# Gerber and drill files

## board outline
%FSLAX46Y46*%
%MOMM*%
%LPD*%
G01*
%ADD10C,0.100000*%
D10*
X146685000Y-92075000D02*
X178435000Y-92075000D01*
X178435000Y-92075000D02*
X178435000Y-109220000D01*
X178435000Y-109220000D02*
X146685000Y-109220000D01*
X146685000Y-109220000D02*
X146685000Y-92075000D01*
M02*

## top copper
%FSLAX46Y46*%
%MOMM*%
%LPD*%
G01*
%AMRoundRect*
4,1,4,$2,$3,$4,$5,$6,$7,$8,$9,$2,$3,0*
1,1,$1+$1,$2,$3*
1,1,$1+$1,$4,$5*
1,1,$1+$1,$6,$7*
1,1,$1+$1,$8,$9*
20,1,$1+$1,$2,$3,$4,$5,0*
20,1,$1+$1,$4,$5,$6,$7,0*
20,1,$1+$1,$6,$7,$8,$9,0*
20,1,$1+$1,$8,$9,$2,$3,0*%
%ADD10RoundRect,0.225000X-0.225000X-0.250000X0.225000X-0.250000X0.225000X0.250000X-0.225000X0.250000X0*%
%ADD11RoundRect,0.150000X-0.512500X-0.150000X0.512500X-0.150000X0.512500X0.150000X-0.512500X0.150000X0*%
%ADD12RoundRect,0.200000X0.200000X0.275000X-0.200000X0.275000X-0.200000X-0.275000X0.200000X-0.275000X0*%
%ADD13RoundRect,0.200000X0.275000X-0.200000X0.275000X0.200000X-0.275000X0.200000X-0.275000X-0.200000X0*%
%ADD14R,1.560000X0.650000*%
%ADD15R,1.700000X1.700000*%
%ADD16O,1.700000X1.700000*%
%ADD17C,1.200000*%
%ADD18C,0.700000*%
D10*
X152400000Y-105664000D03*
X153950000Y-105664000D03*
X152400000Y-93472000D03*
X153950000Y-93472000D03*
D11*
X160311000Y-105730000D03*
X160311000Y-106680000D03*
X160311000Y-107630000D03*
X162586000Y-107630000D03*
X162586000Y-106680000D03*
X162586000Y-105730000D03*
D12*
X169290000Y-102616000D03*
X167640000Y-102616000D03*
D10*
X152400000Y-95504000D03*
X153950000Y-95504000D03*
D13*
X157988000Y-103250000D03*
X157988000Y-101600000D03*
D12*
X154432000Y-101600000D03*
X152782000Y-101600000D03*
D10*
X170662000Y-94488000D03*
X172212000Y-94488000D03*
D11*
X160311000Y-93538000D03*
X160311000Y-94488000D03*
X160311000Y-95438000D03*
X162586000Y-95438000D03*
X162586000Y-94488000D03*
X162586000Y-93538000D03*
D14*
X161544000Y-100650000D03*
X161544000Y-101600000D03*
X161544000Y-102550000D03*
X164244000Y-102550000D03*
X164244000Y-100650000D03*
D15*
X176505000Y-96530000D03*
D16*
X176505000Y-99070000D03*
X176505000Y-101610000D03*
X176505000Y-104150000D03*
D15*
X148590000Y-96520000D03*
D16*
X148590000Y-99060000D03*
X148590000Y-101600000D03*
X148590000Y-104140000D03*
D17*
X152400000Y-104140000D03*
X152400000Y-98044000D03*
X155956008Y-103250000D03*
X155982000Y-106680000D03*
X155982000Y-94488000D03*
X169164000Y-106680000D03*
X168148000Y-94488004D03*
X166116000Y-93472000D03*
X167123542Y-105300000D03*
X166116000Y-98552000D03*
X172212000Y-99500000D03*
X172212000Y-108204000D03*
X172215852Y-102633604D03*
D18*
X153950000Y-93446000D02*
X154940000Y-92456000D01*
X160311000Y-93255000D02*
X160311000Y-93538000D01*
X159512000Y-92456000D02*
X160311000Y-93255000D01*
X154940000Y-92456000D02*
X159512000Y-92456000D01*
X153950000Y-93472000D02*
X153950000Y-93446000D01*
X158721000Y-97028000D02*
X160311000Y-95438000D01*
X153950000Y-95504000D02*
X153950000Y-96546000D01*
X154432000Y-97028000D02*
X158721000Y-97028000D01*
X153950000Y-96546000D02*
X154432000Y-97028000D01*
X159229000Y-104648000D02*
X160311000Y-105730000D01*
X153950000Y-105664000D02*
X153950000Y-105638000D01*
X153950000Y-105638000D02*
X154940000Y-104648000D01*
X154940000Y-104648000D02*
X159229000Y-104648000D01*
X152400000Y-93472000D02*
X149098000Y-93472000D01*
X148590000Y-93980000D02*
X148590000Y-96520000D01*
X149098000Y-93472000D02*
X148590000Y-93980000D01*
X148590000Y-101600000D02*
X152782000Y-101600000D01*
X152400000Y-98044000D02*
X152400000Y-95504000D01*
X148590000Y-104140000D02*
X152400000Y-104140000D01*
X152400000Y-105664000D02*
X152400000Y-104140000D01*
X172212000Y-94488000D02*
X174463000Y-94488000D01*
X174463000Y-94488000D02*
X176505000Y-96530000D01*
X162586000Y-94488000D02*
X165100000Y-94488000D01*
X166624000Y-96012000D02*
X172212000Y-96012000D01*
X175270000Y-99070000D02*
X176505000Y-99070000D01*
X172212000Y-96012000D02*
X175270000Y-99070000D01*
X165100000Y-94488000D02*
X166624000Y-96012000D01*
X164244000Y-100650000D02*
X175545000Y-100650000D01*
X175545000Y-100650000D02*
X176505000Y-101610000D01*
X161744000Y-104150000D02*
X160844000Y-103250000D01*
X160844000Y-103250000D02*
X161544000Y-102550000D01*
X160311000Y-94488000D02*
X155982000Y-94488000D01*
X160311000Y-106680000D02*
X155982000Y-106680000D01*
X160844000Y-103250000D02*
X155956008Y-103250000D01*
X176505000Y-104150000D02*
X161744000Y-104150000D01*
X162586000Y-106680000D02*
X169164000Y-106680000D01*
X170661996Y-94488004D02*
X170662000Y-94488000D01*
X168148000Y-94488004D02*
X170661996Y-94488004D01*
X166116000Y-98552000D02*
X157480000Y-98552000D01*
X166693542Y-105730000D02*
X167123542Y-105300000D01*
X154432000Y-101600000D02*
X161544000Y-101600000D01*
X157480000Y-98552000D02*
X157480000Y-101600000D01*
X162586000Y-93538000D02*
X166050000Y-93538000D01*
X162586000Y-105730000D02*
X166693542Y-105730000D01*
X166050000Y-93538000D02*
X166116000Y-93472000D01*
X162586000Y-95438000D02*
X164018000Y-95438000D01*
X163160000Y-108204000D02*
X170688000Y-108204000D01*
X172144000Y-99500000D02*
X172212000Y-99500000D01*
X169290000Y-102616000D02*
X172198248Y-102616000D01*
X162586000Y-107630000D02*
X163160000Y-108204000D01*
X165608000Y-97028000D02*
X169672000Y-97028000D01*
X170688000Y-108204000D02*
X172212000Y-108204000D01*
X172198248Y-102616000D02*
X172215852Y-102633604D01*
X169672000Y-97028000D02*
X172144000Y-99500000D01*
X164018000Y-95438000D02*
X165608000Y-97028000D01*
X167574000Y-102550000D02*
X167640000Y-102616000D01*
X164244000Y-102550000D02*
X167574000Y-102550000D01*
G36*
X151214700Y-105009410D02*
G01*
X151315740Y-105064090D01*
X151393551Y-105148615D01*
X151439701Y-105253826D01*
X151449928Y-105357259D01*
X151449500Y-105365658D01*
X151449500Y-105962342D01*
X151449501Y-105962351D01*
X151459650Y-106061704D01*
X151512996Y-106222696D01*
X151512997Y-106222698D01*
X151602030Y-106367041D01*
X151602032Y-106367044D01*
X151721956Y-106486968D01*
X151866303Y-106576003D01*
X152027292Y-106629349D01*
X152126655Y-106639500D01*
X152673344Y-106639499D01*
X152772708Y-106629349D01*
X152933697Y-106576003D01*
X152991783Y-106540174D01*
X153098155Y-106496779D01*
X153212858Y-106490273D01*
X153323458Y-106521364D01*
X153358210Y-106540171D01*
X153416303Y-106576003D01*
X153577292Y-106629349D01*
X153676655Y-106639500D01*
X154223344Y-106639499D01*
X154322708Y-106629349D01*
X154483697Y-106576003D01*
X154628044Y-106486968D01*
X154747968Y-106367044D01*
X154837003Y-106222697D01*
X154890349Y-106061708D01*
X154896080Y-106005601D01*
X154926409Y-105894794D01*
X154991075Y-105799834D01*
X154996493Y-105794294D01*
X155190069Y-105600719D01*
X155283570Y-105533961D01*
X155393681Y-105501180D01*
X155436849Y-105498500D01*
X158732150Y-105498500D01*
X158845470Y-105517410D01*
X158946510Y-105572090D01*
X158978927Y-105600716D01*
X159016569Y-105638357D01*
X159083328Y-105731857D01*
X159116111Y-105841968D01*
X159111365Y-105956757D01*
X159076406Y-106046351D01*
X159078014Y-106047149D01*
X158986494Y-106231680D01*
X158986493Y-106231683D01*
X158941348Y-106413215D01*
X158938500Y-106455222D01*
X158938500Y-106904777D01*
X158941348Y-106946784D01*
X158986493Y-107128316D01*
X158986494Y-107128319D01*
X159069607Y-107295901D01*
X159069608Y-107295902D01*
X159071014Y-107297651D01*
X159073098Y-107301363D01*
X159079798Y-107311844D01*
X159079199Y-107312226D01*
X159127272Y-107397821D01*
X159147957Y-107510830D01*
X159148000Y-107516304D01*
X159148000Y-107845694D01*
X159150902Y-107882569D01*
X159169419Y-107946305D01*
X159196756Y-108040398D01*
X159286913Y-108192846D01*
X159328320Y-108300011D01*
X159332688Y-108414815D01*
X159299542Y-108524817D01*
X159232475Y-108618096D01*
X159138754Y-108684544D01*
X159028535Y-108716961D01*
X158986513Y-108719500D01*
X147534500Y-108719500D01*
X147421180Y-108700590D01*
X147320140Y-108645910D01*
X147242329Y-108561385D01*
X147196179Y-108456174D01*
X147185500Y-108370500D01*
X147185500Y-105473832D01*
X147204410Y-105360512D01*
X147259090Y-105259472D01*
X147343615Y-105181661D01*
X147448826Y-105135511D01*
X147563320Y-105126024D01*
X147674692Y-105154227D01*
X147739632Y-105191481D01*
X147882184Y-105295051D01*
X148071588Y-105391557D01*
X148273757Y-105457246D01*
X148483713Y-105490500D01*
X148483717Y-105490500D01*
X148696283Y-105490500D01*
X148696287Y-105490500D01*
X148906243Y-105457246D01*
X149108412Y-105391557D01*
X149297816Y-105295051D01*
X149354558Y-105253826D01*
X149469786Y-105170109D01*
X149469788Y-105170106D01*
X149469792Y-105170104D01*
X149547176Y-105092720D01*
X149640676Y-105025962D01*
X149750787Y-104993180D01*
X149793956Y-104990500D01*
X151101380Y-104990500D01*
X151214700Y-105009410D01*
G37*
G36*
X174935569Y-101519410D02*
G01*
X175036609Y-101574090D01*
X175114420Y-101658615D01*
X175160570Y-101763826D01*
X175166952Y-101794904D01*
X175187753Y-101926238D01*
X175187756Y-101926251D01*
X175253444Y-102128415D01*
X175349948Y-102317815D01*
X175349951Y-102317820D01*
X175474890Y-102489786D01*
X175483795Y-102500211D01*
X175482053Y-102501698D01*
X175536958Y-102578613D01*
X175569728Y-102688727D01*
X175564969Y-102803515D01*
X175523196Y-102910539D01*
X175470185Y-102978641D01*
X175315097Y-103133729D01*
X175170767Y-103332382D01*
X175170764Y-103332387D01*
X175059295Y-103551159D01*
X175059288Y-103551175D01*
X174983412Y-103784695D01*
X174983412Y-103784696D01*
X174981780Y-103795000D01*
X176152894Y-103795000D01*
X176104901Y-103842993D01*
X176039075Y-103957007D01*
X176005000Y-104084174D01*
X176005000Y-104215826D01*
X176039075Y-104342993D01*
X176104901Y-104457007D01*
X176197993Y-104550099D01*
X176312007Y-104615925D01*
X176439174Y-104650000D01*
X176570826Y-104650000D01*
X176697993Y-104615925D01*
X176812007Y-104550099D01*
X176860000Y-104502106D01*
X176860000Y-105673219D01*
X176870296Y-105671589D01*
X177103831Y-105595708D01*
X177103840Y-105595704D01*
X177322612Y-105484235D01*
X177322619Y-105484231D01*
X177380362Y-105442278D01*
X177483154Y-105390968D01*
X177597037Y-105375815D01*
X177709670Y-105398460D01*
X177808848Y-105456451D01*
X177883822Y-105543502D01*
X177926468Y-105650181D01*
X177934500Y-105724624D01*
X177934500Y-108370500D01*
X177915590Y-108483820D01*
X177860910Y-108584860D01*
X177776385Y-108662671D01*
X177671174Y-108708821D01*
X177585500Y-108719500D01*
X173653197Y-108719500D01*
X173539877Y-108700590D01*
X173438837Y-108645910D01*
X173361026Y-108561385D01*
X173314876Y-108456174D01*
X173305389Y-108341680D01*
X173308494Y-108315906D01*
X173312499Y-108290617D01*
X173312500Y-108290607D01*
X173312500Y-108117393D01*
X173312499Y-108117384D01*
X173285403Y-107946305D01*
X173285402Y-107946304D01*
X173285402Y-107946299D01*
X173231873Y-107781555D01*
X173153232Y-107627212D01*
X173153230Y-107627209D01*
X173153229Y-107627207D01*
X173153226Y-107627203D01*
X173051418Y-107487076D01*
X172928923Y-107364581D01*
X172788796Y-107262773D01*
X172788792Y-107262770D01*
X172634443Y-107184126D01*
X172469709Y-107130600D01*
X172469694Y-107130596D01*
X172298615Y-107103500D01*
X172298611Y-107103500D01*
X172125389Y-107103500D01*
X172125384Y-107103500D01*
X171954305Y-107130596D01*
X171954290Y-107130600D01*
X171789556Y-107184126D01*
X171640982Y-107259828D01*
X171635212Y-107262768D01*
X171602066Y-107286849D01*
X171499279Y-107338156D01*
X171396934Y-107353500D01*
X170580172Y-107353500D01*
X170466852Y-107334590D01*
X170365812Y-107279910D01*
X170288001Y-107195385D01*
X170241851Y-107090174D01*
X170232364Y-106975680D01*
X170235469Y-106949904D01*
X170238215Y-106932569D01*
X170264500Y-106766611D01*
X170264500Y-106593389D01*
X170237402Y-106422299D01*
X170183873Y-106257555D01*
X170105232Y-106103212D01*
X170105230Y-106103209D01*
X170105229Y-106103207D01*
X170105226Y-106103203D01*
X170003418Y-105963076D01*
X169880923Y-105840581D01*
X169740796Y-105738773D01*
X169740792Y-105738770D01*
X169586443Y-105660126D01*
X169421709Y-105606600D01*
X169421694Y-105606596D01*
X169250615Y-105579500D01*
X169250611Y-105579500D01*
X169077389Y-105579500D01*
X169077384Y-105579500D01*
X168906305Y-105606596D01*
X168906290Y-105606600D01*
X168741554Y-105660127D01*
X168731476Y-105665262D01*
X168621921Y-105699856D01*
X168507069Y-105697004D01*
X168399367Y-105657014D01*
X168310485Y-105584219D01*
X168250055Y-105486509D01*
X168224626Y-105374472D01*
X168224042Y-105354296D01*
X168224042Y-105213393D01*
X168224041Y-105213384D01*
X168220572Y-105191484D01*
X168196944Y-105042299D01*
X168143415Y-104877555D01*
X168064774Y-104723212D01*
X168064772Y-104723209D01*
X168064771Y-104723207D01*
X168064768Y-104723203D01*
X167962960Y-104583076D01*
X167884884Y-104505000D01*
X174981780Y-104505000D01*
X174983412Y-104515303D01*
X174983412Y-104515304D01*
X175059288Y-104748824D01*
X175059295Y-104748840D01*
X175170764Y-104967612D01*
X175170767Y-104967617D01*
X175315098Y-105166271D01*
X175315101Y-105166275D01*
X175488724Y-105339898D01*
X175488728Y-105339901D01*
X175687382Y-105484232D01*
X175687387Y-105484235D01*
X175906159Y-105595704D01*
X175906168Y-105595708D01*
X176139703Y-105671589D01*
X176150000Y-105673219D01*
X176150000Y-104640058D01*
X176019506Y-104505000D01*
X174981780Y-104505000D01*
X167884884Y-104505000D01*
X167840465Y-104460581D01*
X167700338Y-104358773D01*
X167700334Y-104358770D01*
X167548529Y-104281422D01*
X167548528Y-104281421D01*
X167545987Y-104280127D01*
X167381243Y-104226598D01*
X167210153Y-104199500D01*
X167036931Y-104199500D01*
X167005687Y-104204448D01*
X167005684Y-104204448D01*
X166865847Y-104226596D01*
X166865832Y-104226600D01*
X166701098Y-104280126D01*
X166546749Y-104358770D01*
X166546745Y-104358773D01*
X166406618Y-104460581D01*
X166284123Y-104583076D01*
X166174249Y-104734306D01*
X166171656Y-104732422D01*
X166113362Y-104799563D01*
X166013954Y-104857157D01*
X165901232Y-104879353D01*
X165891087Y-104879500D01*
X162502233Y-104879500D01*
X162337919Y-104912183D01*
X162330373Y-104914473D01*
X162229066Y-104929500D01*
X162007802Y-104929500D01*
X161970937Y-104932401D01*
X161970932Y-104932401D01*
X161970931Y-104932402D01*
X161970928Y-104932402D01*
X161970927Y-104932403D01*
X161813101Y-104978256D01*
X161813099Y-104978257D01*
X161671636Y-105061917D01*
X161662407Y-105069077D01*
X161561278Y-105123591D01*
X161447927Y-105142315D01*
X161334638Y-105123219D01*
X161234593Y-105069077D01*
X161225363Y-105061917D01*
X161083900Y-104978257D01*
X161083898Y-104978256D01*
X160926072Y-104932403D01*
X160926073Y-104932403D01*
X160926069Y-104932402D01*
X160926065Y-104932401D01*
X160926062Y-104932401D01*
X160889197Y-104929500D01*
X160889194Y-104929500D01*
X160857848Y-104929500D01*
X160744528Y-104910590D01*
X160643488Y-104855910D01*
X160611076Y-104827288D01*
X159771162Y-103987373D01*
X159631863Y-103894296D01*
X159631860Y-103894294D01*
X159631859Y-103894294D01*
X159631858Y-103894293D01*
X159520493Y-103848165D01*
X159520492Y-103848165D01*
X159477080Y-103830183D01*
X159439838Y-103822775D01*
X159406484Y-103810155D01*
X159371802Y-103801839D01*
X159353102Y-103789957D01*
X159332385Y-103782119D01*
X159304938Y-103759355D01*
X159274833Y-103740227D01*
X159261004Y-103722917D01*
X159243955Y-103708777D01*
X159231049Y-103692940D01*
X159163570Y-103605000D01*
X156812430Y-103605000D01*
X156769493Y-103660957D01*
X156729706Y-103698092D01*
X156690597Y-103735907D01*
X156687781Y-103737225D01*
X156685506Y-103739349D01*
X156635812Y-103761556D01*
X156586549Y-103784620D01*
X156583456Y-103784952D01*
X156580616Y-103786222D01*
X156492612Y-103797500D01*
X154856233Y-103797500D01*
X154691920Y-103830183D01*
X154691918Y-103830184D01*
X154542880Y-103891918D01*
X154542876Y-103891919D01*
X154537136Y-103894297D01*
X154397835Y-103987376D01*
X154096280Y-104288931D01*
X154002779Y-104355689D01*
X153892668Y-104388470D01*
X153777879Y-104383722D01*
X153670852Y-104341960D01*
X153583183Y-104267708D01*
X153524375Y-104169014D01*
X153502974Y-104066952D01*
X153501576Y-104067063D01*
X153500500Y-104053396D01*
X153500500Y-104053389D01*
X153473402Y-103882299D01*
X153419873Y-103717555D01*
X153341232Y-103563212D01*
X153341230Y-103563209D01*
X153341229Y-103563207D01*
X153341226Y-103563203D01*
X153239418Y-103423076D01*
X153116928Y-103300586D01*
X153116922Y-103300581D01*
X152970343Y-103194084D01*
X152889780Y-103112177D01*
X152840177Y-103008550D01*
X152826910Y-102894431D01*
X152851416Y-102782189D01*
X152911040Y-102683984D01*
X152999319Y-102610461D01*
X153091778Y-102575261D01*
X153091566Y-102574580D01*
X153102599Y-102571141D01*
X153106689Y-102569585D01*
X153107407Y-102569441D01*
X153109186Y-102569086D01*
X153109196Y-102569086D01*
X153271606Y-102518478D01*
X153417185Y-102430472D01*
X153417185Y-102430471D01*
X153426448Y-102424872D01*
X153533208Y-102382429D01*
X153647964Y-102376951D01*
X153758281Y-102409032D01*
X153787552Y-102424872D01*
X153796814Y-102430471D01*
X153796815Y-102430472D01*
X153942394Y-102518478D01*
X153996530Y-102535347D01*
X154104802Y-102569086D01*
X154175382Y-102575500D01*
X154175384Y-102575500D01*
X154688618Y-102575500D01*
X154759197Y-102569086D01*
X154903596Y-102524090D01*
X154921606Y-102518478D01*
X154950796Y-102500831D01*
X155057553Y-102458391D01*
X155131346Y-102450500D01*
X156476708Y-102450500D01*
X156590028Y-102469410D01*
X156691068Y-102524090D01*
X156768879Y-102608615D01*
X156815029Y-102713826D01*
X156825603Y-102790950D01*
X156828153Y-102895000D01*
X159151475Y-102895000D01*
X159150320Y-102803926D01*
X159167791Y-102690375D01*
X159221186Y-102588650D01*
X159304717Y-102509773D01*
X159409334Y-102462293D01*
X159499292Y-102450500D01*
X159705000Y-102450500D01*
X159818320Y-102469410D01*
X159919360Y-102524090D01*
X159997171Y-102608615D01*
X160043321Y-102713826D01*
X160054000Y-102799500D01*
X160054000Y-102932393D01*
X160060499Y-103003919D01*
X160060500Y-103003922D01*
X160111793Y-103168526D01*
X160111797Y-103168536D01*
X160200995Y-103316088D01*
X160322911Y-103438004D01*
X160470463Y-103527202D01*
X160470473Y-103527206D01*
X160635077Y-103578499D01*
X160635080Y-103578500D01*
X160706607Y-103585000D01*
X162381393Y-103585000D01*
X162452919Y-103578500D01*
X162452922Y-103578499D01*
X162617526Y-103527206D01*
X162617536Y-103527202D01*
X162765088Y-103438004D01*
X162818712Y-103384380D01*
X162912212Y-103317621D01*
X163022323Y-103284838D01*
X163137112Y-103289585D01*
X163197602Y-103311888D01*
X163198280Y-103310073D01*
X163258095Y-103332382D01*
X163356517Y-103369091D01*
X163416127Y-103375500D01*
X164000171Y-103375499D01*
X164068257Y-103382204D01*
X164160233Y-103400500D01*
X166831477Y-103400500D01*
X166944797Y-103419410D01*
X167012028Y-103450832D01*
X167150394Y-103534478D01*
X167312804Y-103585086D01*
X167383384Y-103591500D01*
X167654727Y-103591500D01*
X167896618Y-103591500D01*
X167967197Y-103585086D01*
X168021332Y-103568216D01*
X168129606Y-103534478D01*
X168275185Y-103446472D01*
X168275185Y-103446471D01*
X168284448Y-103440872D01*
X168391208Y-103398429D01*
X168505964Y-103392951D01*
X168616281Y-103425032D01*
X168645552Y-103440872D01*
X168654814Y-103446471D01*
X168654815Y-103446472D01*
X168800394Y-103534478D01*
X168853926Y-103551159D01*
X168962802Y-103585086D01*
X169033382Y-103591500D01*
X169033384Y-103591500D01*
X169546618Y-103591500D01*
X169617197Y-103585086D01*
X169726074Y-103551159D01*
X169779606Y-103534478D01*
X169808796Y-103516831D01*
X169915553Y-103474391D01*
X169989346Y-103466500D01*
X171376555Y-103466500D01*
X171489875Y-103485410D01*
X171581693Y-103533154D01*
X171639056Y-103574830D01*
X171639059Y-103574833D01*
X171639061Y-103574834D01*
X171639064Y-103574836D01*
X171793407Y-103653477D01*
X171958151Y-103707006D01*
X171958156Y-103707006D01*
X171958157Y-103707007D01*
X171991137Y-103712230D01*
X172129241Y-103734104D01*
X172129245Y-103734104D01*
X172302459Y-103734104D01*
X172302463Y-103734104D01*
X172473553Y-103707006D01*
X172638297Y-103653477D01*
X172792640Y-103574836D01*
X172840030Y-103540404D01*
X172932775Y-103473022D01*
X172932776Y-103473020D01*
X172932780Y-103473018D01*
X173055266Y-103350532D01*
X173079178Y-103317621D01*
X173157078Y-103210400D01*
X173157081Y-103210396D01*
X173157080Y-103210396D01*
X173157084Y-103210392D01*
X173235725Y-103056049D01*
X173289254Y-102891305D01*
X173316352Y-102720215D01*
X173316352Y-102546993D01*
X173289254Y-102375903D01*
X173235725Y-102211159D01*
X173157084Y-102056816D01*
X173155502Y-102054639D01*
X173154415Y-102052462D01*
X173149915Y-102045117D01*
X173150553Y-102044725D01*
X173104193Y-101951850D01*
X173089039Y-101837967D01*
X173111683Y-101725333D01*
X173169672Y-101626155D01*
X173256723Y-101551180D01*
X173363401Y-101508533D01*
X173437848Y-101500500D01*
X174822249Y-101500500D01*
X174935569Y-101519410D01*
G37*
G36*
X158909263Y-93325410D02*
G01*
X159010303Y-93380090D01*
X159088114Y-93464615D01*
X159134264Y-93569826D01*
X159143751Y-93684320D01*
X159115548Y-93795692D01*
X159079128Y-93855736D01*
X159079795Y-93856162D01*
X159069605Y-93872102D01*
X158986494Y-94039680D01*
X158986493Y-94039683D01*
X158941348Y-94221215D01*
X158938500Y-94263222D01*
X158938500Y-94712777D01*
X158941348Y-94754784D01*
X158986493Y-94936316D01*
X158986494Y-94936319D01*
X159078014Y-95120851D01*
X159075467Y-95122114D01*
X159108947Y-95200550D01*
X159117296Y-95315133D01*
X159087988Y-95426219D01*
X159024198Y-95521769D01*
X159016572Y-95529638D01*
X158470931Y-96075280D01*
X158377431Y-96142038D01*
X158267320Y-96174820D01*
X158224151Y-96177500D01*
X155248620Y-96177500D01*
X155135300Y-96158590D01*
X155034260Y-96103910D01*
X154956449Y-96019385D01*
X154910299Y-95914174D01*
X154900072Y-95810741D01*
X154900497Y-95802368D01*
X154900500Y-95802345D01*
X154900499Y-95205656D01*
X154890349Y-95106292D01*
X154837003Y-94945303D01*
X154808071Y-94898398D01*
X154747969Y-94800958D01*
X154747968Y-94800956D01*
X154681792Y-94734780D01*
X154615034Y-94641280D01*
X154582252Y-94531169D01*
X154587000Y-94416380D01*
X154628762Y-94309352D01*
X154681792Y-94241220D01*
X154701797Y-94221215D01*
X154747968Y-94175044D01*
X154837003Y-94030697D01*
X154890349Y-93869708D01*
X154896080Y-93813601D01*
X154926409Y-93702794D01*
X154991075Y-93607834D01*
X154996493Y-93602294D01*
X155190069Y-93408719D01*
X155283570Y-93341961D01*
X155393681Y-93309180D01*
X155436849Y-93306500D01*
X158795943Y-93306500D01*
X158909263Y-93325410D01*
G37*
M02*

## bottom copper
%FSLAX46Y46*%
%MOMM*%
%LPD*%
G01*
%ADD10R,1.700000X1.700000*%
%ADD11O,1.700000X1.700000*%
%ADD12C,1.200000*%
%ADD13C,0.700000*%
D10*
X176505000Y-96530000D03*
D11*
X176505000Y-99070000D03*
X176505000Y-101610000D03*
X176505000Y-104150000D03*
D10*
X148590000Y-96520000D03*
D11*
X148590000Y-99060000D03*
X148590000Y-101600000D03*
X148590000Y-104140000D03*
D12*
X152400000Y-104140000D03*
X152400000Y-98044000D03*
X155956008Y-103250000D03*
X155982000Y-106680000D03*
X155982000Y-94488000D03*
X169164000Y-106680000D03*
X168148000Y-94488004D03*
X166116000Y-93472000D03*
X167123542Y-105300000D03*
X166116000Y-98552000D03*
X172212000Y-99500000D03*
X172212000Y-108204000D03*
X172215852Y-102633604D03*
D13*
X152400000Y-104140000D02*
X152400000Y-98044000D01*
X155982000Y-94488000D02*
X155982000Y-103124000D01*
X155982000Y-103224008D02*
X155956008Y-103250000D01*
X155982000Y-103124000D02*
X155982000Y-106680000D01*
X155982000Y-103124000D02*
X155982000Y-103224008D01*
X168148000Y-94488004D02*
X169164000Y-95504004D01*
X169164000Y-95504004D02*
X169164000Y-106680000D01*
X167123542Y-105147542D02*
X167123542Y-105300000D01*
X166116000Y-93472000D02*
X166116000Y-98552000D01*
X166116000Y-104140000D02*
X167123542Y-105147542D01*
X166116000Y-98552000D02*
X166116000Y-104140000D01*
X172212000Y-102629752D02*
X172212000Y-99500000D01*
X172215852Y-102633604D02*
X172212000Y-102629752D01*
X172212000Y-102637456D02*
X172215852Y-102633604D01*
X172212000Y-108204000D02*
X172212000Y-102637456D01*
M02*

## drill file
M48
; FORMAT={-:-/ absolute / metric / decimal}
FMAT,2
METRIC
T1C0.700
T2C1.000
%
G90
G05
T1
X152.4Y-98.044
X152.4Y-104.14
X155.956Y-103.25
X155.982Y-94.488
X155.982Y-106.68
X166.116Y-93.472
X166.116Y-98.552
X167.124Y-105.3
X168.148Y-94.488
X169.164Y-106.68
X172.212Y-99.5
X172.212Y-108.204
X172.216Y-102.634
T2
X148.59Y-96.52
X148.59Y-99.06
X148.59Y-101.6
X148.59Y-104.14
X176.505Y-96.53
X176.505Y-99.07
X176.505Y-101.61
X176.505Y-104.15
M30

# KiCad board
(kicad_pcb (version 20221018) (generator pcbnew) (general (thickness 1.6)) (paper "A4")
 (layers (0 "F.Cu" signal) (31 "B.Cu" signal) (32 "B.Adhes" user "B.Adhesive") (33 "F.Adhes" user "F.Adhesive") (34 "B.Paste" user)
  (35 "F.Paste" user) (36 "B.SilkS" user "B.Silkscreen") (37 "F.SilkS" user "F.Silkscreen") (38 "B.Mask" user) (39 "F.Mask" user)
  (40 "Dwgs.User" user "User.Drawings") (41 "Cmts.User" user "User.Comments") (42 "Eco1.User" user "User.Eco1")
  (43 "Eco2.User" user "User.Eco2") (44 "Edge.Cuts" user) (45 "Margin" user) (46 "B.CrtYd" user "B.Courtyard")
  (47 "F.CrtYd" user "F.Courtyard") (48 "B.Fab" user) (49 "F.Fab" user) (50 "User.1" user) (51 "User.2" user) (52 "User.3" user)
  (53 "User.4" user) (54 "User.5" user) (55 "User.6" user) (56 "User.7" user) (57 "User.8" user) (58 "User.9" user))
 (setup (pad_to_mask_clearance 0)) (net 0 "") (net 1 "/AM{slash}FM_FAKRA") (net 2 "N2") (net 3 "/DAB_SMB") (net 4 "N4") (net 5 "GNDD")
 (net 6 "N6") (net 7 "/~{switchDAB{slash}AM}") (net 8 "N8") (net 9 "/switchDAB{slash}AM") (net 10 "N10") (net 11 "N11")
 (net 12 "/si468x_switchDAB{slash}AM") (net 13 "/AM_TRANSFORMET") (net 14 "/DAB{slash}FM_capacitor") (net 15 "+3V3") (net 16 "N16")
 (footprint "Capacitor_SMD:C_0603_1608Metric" (layer "F.Cu") (at 153.175 105.664)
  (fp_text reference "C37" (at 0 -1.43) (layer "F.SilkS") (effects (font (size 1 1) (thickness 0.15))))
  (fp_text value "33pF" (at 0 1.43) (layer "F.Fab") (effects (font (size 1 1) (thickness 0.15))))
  (pad "1" smd roundrect (at -0.775 0) (size 0.9 0.95) (layers "F.Cu" "F.Paste" "F.Mask") (roundrect_rratio 0.25)
   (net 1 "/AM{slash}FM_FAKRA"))
  (pad "2" smd roundrect (at 0.775 0) (size 0.9 0.95) (layers "F.Cu" "F.Paste" "F.Mask") (roundrect_rratio 0.25) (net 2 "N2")))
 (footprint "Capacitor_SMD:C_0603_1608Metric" (layer "F.Cu") (at 153.175 93.472)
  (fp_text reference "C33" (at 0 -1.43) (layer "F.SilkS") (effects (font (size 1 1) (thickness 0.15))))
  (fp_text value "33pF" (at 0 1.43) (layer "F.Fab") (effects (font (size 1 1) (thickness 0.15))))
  (pad "1" smd roundrect (at -0.775 0) (size 0.9 0.95) (layers "F.Cu" "F.Paste" "F.Mask") (roundrect_rratio 0.25) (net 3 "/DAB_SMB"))
  (pad "2" smd roundrect (at 0.775 0) (size 0.9 0.95) (layers "F.Cu" "F.Paste" "F.Mask") (roundrect_rratio 0.25) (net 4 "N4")))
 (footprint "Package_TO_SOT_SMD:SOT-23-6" (layer "F.Cu") (at 161.4485 106.68)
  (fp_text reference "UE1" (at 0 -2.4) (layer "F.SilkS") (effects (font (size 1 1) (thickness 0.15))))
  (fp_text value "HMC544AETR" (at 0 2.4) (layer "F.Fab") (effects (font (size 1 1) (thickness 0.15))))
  (pad "1" smd roundrect (at -1.1375 -0.95) (size 1.325 0.6) (layers "F.Cu" "F.Paste" "F.Mask") (roundrect_rratio 0.25) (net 2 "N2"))
  (pad "2" smd roundrect (at -1.1375 0) (size 1.325 0.6) (layers "F.Cu" "F.Paste" "F.Mask") (roundrect_rratio 0.25) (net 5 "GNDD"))
  (pad "3" smd roundrect (at -1.1375 0.95) (size 1.325 0.6) (layers "F.Cu" "F.Paste" "F.Mask") (roundrect_rratio 0.25) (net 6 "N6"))
  (pad "4" smd roundrect (at 1.1375 0.95) (size 1.325 0.6) (layers "F.Cu" "F.Paste" "F.Mask") (roundrect_rratio 0.25)
   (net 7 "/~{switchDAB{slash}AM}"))
  (pad "5" smd roundrect (at 1.1375 0) (size 1.325 0.6) (layers "F.Cu" "F.Paste" "F.Mask") (roundrect_rratio 0.25) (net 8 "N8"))
  (pad "6" smd roundrect (at 1.1375 -0.95) (size 1.325 0.6) (layers "F.Cu" "F.Paste" "F.Mask") (roundrect_rratio 0.25)
   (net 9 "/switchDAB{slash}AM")))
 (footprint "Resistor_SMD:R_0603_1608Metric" (layer "F.Cu") (at 168.465 102.616 180)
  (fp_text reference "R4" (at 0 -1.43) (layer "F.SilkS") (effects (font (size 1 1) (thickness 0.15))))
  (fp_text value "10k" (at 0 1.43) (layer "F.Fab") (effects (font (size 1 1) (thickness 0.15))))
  (pad "1" smd roundrect (at -0.825 0 180) (size 0.8 0.95) (layers "F.Cu" "F.Paste" "F.Mask") (roundrect_rratio 0.25)
   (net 7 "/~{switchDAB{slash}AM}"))
  (pad "2" smd roundrect (at 0.825 0 180) (size 0.8 0.95) (layers "F.Cu" "F.Paste" "F.Mask") (roundrect_rratio 0.25) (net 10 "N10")))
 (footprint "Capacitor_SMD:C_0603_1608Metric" (layer "F.Cu") (at 153.175 95.504)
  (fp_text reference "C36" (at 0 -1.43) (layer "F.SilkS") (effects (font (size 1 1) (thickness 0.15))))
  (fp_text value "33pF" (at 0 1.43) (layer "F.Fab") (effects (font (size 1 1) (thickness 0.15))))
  (pad "1" smd roundrect (at -0.775 0) (size 0.9 0.95) (layers "F.Cu" "F.Paste" "F.Mask") (roundrect_rratio 0.25)
   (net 1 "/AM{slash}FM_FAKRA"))
  (pad "2" smd roundrect (at 0.775 0) (size 0.9 0.95) (layers "F.Cu" "F.Paste" "F.Mask") (roundrect_rratio 0.25) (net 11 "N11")))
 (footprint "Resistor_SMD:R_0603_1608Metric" (layer "F.Cu") (at 157.988 102.425 90)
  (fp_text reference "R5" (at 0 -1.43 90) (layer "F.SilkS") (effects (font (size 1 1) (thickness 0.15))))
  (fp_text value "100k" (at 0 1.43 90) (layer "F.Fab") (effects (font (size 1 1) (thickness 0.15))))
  (pad "1" smd roundrect (at -0.825 0 90) (size 0.8 0.95) (layers "F.Cu" "F.Paste" "F.Mask") (roundrect_rratio 0.25) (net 5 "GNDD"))
  (pad "2" smd roundrect (at 0.825 0 90) (size 0.8 0.95) (layers "F.Cu" "F.Paste" "F.Mask") (roundrect_rratio 0.25)
   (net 9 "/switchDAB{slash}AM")))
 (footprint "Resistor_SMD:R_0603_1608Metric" (layer "F.Cu") (at 153.607 101.6 180)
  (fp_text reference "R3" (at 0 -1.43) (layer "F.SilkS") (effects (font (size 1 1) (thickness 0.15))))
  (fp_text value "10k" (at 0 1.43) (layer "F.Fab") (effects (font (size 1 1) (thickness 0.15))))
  (pad "1" smd roundrect (at -0.825 0 180) (size 0.8 0.95) (layers "F.Cu" "F.Paste" "F.Mask") (roundrect_rratio 0.25)
   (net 9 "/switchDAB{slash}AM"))
  (pad "2" smd roundrect (at 0.825 0 180) (size 0.8 0.95) (layers "F.Cu" "F.Paste" "F.Mask") (roundrect_rratio 0.25)
   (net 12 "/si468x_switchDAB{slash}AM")))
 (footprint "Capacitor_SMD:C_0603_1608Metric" (layer "F.Cu") (at 171.437 94.488)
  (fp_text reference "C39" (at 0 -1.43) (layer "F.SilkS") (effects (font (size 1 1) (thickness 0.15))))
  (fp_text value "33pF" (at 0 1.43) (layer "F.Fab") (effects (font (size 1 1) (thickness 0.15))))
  (pad "1" smd roundrect (at -0.775 0) (size 0.9 0.95) (layers "F.Cu" "F.Paste" "F.Mask") (roundrect_rratio 0.25) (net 8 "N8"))
  (pad "2" smd roundrect (at 0.775 0) (size 0.9 0.95) (layers "F.Cu" "F.Paste" "F.Mask") (roundrect_rratio 0.25) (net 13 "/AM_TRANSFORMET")))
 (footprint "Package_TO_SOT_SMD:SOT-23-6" (layer "F.Cu") (at 161.4485 94.488)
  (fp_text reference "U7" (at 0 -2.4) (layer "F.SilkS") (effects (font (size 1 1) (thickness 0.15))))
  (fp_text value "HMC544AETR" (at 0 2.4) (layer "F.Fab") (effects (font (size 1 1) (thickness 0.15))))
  (pad "1" smd roundrect (at -1.1375 -0.95) (size 1.325 0.6) (layers "F.Cu" "F.Paste" "F.Mask") (roundrect_rratio 0.25) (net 4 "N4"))
  (pad "2" smd roundrect (at -1.1375 0) (size 1.325 0.6) (layers "F.Cu" "F.Paste" "F.Mask") (roundrect_rratio 0.25) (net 5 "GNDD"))
  (pad "3" smd roundrect (at -1.1375 0.95) (size 1.325 0.6) (layers "F.Cu" "F.Paste" "F.Mask") (roundrect_rratio 0.25) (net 11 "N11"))
  (pad "4" smd roundrect (at 1.1375 0.95) (size 1.325 0.6) (layers "F.Cu" "F.Paste" "F.Mask") (roundrect_rratio 0.25)
   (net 7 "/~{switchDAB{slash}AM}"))
  (pad "5" smd roundrect (at 1.1375 0) (size 1.325 0.6) (layers "F.Cu" "F.Paste" "F.Mask") (roundrect_rratio 0.25)
   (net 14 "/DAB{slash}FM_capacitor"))
  (pad "6" smd roundrect (at 1.1375 -0.95) (size 1.325 0.6) (layers "F.Cu" "F.Paste" "F.Mask") (roundrect_rratio 0.25)
   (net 9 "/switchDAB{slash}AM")))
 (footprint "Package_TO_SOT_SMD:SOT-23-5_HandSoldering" (layer "F.Cu") (at 162.894 101.6)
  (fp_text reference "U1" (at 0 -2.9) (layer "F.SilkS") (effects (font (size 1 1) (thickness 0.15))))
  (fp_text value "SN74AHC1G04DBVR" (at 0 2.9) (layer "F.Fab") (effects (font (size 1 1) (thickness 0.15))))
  (pad "1" smd rect (at -1.35 -0.95) (size 1.56 0.65) (layers "F.Cu" "F.Paste" "F.Mask"))
  (pad "2" smd rect (at -1.35 0) (size 1.56 0.65) (layers "F.Cu" "F.Paste" "F.Mask") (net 9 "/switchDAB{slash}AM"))
  (pad "3" smd rect (at -1.35 0.95) (size 1.56 0.65) (layers "F.Cu" "F.Paste" "F.Mask") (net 5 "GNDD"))
  (pad "4" smd rect (at 1.35 0.95) (size 1.56 0.65) (layers "F.Cu" "F.Paste" "F.Mask") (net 10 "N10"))
  (pad "5" smd rect (at 1.35 -0.95) (size 1.56 0.65) (layers "F.Cu" "F.Paste" "F.Mask") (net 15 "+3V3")))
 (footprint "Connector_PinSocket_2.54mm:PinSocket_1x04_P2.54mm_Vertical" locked (layer "B.Cu") (at 176.505 96.53 180)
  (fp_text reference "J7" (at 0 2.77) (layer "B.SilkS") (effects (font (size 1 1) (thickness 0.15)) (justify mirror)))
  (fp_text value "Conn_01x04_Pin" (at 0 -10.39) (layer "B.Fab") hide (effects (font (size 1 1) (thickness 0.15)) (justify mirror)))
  (pad "1" thru_hole rect locked (at 0 0 180) (size 1.7 1.7) (drill 1) (layers "*.Cu" "*.Mask") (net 13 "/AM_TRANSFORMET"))
  (pad "2" thru_hole oval locked (at 0 -2.54 180) (size 1.7 1.7) (drill 1) (layers "*.Cu" "*.Mask") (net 14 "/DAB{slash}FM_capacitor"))
  (pad "3" thru_hole oval locked (at 0 -5.08 180) (size 1.7 1.7) (drill 1) (layers "*.Cu" "*.Mask") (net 15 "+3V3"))
  (pad "4" thru_hole oval locked (at 0 -7.62 180) (size 1.7 1.7) (drill 1) (layers "*.Cu" "*.Mask") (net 5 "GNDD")))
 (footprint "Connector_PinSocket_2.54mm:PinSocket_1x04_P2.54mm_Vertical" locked (layer "B.Cu") (at 148.59 96.52 180)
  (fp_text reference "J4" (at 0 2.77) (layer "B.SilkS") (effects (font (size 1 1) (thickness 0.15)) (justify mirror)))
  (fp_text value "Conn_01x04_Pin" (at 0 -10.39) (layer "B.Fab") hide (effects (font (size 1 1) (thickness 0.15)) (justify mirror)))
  (pad "1" thru_hole rect locked (at 0 0 180) (size 1.7 1.7) (drill 1) (layers "*.Cu" "*.Mask") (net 3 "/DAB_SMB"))
  (pad "2" thru_hole oval locked (at 0 -2.54 180) (size 1.7 1.7) (drill 1) (layers "*.Cu" "*.Mask") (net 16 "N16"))
  (pad "3" thru_hole oval locked (at 0 -5.08 180) (size 1.7 1.7) (drill 1) (layers "*.Cu" "*.Mask") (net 12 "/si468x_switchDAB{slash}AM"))
  (pad "4" thru_hole oval locked (at 0 -7.62 180) (size 1.7 1.7) (drill 1) (layers "*.Cu" "*.Mask") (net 1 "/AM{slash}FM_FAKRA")))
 (gr_line (start 146.685 92.075) (end 178.435 92.075) (stroke (width 0.1) (type default)) (layer "Edge.Cuts"))
 (gr_line (start 178.435 92.075) (end 178.435 109.22) (stroke (width 0.1) (type default)) (layer "Edge.Cuts"))
 (gr_line (start 178.435 109.22) (end 146.685 109.22) (stroke (width 0.1) (type default)) (layer "Edge.Cuts"))
 (gr_line (start 146.685 109.22) (end 146.685 92.075) (stroke (width 0.1) (type default)) (layer "Edge.Cuts"))
 (segment (start 153.95 93.446) (end 154.94 92.456) (width 0.7) (layer "F.Cu") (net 4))
 (segment (start 160.311 93.255) (end 160.311 93.538) (width 0.7) (layer "F.Cu") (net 4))
 (segment (start 159.512 92.456) (end 160.311 93.255) (width 0.7) (layer "F.Cu") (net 4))
 (segment (start 154.94 92.456) (end 159.512 92.456) (width 0.7) (layer "F.Cu") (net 4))
 (segment (start 153.95 93.472) (end 153.95 93.446) (width 0.7) (layer "F.Cu") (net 4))
 (segment (start 158.721 97.028) (end 160.311 95.438) (width 0.7) (layer "F.Cu") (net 11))
 (segment (start 153.95 95.504) (end 153.95 96.546) (width 0.7) (layer "F.Cu") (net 11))
 (segment (start 154.432 97.028) (end 158.721 97.028) (width 0.7) (layer "F.Cu") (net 11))
 (segment (start 153.95 96.546) (end 154.432 97.028) (width 0.7) (layer "F.Cu") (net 11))
 (segment (start 159.229 104.648) (end 160.311 105.73) (width 0.7) (layer "F.Cu") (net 2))
 (segment (start 153.95 105.664) (end 153.95 105.638) (width 0.7) (layer "F.Cu") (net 2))
 (segment (start 153.95 105.638) (end 154.94 104.648) (width 0.7) (layer "F.Cu") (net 2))
 (segment (start 154.94 104.648) (end 159.229 104.648) (width 0.7) (layer "F.Cu") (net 2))
 (segment (start 152.4 93.472) (end 149.098 93.472) (width 0.7) (layer "F.Cu") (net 3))
 (segment (start 148.59 93.98) (end 148.59 96.52) (width 0.7) (layer "F.Cu") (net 3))
 (segment (start 149.098 93.472) (end 148.59 93.98) (width 0.7) (layer "F.Cu") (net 3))
 (segment (start 148.59 101.6) (end 152.782 101.6) (width 0.7) (layer "F.Cu") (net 12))
 (segment (start 152.4 98.044) (end 152.4 95.504) (width 0.7) (layer "F.Cu") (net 1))
 (segment (start 148.59 104.14) (end 152.4 104.14) (width 0.7) (layer "F.Cu") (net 1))
 (segment (start 152.4 105.664) (end 152.4 104.14) (width 0.7) (layer "F.Cu") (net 1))
 (via (at 152.4 104.14) (size 1.2) (drill 0.7) (layers "F.Cu" "B.Cu") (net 1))
 (via (at 152.4 98.044) (size 1.2) (drill 0.7) (layers "F.Cu" "B.Cu") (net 1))
 (segment (start 152.4 104.14) (end 152.4 98.044) (width 0.7) (layer "B.Cu") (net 1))
 (segment (start 172.212 94.488) (end 174.463 94.488) (width 0.7) (layer "F.Cu") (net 13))
 (segment (start 174.463 94.488) (end 176.505 96.53) (width 0.7) (layer "F.Cu") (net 13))
 (segment (start 162.586 94.488) (end 165.1 94.488) (width 0.7) (layer "F.Cu") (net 14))
 (segment (start 166.624 96.012) (end 172.212 96.012) (width 0.7) (layer "F.Cu") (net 14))
 (segment (start 175.27 99.07) (end 176.505 99.07) (width 0.7) (layer "F.Cu") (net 14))
 (segment (start 172.212 96.012) (end 175.27 99.07) (width 0.7) (layer "F.Cu") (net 14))
 (segment (start 165.1 94.488) (end 166.624 96.012) (width 0.7) (layer "F.Cu") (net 14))
 (segment (start 164.244 100.65) (end 175.545 100.65) (width 0.7) (layer "F.Cu") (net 15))
 (segment (start 175.545 100.65) (end 176.505 101.61) (width 0.7) (layer "F.Cu") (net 15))
 (segment (start 161.744 104.15) (end 160.844 103.25) (width 0.7) (layer "F.Cu") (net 5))
 (segment (start 160.844 103.25) (end 161.544 102.55) (width 0.7) (layer "F.Cu") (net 5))
 (segment (start 160.311 94.488) (end 155.982 94.488) (width 0.7) (layer "F.Cu") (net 5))
 (segment (start 160.311 106.68) (end 155.982 106.68) (width 0.7) (layer "F.Cu") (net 5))
 (segment (start 160.844 103.25) (end 155.956008 103.25) (width 0.7) (layer "F.Cu") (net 5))
 (segment (start 176.505 104.15) (end 161.744 104.15) (width 0.7) (layer "F.Cu") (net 5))
 (via (at 155.956008 103.25) (size 1.2) (drill 0.7) (layers "F.Cu" "B.Cu") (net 5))
 (via (at 155.982 106.68) (size 1.2) (drill 0.7) (layers "F.Cu" "B.Cu") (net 5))
 (via (at 155.982 94.488) (size 1.2) (drill 0.7) (layers "F.Cu" "B.Cu") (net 5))
 (segment (start 155.982 94.488) (end 155.982 103.124) (width 0.7) (layer "B.Cu") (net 5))
 (segment (start 155.982 103.224008) (end 155.956008 103.25) (width 0.7) (layer "B.Cu") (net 5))
 (segment (start 155.982 103.124) (end 155.982 106.68) (width 0.7) (layer "B.Cu") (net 5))
 (segment (start 155.982 103.124) (end 155.982 103.224008) (width 0.7) (layer "B.Cu") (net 5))
 (segment (start 162.586 106.68) (end 169.164 106.68) (width 0.7) (layer "F.Cu") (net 8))
 (segment (start 170.661996 94.488004) (end 170.662 94.488) (width 0.7) (layer "F.Cu") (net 8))
 (segment (start 168.148 94.488004) (end 170.661996 94.488004) (width 0.7) (layer "F.Cu") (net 8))
 (via (at 169.164 106.68) (size 1.2) (drill 0.7) (layers "F.Cu" "B.Cu") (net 8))
 (via (at 168.148 94.488004) (size 1.2) (drill 0.7) (layers "F.Cu" "B.Cu") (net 8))
 (segment (start 168.148 94.488004) (end 169.164 95.504004) (width 0.7) (layer "B.Cu") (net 8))
 (segment (start 169.164 95.504004) (end 169.164 106.68) (width 0.7) (layer "B.Cu") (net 8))
 (segment (start 166.116 98.552) (end 157.48 98.552) (width 0.7) (layer "F.Cu") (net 9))
 (segment (start 166.693542 105.73) (end 167.123542 105.3) (width 0.7) (layer "F.Cu") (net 9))
 (segment (start 154.432 101.6) (end 161.544 101.6) (width 0.7) (layer "F.Cu") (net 9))
 (segment (start 157.48 98.552) (end 157.48 101.6) (width 0.7) (layer "F.Cu") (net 9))
 (segment (start 162.586 93.538) (end 166.05 93.538) (width 0.7) (layer "F.Cu") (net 9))
 (segment (start 162.586 105.73) (end 166.693542 105.73) (width 0.7) (layer "F.Cu") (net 9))
 (segment (start 166.05 93.538) (end 166.116 93.472) (width 0.7) (layer "F.Cu") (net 9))
 (via (at 166.116 93.472) (size 1.2) (drill 0.7) (layers "F.Cu" "B.Cu") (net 9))
 (via (at 167.123542 105.3) (size 1.2) (drill 0.7) (layers "F.Cu" "B.Cu") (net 9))
 (via (at 166.116 98.552) (size 1.2) (drill 0.7) (layers "F.Cu" "B.Cu") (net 9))
 (segment (start 167.123542 105.147542) (end 167.123542 105.3) (width 0.7) (layer "B.Cu") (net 9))
 (segment (start 166.116 93.472) (end 166.116 98.552) (width 0.7) (layer "B.Cu") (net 9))
 (segment (start 166.116 104.14) (end 167.123542 105.147542) (width 0.7) (layer "B.Cu") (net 9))
 (segment (start 166.116 98.552) (end 166.116 104.14) (width 0.7) (layer "B.Cu") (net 9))
 (segment (start 162.586 95.438) (end 164.018 95.438) (width 0.7) (layer "F.Cu") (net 7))
 (segment (start 163.16 108.204) (end 170.688 108.204) (width 0.7) (layer "F.Cu") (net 7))
 (segment (start 172.144 99.5) (end 172.212 99.5) (width 0.7) (layer "F.Cu") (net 7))
 (segment (start 169.29 102.616) (end 172.198248 102.616) (width 0.7) (layer "F.Cu") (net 7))
 (segment (start 162.586 107.63) (end 163.16 108.204) (width 0.7) (layer "F.Cu") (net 7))
 (segment (start 165.608 97.028) (end 169.672 97.028) (width 0.7) (layer "F.Cu") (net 7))
 (segment (start 170.688 108.204) (end 172.212 108.204) (width 0.7) (layer "F.Cu") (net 7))
 (segment (start 172.198248 102.616) (end 172.215852 102.633604) (width 0.7) (layer "F.Cu") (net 7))
 (segment (start 169.672 97.028) (end 172.144 99.5) (width 0.7) (layer "F.Cu") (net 7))
 (segment (start 164.018 95.438) (end 165.608 97.028) (width 0.7) (layer "F.Cu") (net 7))
 (via (at 172.212 99.5) (size 1.2) (drill 0.7) (layers "F.Cu" "B.Cu") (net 7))
 (via (at 172.212 108.204) (size 1.2) (drill 0.7) (layers "F.Cu" "B.Cu") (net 7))
 (via (at 172.215852 102.633604) (size 1.2) (drill 0.7) (layers "F.Cu" "B.Cu") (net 7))
 (segment (start 172.212 102.629752) (end 172.212 99.5) (width 0.7) (layer "B.Cu") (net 7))
 (segment (start 172.215852 102.633604) (end 172.212 102.629752) (width 0.7) (layer "B.Cu") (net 7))
 (segment (start 172.212 102.637456) (end 172.215852 102.633604) (width 0.7) (layer "B.Cu") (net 7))
 (segment (start 172.212 108.204) (end 172.212 102.637456) (width 0.7) (layer "B.Cu") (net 7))
 (segment (start 167.574 102.55) (end 167.64 102.616) (width 0.7) (layer "F.Cu") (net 10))
 (segment (start 164.244 102.55) (end 167.574 102.55) (width 0.7) (layer "F.Cu") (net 10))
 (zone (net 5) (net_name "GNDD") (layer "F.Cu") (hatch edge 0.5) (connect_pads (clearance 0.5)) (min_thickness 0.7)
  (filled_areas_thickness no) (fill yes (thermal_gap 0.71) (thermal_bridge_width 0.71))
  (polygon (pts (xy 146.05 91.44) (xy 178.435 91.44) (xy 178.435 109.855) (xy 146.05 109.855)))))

